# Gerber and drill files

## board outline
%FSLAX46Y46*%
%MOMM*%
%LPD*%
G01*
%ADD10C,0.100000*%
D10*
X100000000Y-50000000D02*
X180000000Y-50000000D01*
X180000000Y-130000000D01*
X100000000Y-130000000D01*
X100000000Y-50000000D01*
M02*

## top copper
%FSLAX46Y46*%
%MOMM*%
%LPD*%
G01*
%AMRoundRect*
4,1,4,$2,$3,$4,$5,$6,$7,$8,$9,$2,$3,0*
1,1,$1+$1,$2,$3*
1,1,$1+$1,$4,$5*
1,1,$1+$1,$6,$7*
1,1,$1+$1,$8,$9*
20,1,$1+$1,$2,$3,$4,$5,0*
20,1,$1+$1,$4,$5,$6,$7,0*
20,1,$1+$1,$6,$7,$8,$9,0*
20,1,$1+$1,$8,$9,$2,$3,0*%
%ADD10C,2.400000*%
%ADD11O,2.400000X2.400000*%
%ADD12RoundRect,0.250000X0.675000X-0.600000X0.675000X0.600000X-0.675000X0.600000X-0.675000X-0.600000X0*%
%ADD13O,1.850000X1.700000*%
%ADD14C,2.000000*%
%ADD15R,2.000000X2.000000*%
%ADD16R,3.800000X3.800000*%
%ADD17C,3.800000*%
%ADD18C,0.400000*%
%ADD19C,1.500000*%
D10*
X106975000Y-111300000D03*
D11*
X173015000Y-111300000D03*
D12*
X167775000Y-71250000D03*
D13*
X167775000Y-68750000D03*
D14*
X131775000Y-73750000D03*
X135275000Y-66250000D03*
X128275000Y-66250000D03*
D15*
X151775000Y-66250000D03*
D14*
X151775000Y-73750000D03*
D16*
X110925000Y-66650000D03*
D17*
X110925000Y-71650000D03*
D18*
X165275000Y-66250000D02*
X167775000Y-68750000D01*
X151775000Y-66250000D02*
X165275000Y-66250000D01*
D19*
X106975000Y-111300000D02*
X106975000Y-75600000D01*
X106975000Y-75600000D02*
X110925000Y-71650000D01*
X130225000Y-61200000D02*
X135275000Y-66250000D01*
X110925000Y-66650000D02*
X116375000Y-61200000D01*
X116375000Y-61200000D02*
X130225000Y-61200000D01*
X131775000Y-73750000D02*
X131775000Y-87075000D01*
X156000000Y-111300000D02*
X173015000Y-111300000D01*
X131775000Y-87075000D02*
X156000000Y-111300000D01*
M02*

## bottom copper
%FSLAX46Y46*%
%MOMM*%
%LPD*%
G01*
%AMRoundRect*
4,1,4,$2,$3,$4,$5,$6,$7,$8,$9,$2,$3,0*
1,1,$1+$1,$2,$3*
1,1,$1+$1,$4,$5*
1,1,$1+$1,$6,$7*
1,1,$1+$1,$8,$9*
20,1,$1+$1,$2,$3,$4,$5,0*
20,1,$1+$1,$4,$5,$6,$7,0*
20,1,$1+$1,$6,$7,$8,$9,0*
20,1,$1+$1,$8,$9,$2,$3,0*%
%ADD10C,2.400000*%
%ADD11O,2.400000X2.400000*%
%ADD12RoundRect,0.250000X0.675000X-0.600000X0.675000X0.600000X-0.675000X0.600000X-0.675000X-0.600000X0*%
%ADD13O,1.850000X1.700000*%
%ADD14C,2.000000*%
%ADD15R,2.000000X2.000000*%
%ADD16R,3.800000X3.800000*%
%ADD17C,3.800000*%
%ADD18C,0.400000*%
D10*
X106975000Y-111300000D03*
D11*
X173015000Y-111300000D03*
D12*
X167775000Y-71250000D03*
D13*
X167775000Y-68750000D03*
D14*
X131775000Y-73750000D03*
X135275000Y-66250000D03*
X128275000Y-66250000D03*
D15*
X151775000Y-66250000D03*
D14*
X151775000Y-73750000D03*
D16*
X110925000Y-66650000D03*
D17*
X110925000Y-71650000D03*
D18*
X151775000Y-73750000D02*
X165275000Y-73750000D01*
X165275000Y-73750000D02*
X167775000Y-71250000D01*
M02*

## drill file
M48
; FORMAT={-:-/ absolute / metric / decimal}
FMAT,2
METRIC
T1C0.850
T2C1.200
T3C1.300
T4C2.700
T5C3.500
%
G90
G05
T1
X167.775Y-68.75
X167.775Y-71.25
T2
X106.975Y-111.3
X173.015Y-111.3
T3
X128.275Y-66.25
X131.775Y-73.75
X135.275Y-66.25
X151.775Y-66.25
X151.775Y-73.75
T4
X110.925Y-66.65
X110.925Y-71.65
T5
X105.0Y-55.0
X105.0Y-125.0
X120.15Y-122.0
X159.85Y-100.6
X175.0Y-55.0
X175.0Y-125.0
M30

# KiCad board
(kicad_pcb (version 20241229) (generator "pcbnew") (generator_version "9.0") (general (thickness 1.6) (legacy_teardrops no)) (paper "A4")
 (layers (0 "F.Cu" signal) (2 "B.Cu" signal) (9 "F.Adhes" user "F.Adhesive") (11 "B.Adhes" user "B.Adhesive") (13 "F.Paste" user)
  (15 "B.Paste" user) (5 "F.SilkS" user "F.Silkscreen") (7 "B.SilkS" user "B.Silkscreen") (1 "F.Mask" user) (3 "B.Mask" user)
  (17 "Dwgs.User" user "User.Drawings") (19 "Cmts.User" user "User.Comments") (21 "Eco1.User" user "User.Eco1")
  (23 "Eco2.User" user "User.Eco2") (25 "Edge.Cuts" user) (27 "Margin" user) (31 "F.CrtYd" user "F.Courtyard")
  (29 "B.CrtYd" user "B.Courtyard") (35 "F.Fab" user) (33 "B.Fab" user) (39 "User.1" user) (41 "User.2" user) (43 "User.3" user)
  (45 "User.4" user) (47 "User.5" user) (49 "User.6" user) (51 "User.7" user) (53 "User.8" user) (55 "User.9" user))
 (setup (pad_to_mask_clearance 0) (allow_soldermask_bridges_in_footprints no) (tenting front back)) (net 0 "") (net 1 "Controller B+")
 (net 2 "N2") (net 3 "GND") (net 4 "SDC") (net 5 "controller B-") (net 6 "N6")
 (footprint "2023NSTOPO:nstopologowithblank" (layer "F.Cu") (at 154.9 81.3)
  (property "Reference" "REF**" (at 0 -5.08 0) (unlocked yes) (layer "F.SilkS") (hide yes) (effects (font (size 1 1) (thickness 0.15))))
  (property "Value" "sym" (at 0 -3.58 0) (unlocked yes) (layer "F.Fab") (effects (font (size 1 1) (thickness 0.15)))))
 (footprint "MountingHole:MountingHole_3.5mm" (layer "F.Cu") (at 175 125)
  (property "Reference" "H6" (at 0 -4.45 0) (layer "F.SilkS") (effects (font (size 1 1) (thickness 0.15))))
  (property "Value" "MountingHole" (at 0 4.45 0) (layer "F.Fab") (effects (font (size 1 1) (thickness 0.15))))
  (pad "" np_thru_hole circle (at 0 0) (size 3.5 3.5) (drill 3.5) (layers "*.Cu" "*.Mask")))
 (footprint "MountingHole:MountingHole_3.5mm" (layer "F.Cu") (at 159.85 100.6)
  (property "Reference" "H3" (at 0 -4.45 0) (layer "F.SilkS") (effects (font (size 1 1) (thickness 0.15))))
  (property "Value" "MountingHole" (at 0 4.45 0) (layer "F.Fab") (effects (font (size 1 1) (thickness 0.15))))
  (pad "" np_thru_hole circle (at 0 0) (size 3.5 3.5) (drill 3.5) (layers "*.Cu" "*.Mask")))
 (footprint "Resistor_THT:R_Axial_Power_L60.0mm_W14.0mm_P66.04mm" (layer "F.Cu") (at 106.975 111.3)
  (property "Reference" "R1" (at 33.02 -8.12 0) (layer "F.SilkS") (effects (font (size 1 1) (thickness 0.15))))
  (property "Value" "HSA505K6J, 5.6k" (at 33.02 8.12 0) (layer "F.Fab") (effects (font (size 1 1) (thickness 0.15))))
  (pad "1" thru_hole circle (at 0 0) (size 2.4 2.4) (drill 1.2) (layers "*.Cu" "*.Mask") (remove_unused_layers no) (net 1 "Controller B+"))
  (pad "2" thru_hole oval (at 66.04 0) (size 2.4 2.4) (drill 1.2) (layers "*.Cu" "*.Mask") (remove_unused_layers no) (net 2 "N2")))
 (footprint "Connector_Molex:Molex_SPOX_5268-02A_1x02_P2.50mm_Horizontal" (layer "F.Cu") (at 167.775 71.25 90)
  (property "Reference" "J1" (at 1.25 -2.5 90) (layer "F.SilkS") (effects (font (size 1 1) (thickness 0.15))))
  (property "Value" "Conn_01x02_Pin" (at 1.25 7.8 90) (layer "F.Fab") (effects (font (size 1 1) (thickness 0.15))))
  (pad "1" thru_hole roundrect (at 0 0 90) (size 1.7 1.85) (drill 0.85) (layers "*.Cu" "*.Mask") (remove_unused_layers no)
   (roundrect_rratio 0.147059) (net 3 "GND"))
  (pad "2" thru_hole oval (at 2.5 0 90) (size 1.7 1.85) (drill 0.85) (layers "*.Cu" "*.Mask") (remove_unused_layers no) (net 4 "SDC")))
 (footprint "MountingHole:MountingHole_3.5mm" (layer "F.Cu") (at 105 125)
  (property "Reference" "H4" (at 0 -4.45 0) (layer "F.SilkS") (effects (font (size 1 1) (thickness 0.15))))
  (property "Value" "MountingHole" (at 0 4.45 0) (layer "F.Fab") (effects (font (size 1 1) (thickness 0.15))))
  (pad "" np_thru_hole circle (at 0 0) (size 3.5 3.5) (drill 3.5) (layers "*.Cu" "*.Mask")))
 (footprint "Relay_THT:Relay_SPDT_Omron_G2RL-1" (layer "F.Cu") (at 151.775 66.25 -90)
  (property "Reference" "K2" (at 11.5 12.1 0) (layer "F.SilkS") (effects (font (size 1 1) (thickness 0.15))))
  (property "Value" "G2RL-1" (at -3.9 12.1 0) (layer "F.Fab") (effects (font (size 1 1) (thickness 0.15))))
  (pad "11" thru_hole circle (at 7.5 20 270) (size 2 2) (drill 1.3) (layers "*.Cu" "*.Mask") (remove_unused_layers no) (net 2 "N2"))
  (pad "12" thru_hole circle (at 0 16.5 270) (size 2 2) (drill 1.3) (layers "*.Cu" "*.Mask") (remove_unused_layers no)
   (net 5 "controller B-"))
  (pad "14" thru_hole circle (at 0 23.5 270) (size 2 2) (drill 1.3) (layers "*.Cu" "*.Mask") (remove_unused_layers no) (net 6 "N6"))
  (pad "A1" thru_hole rect (at 0 0 270) (size 2 2) (drill 1.3) (layers "*.Cu" "*.Mask") (remove_unused_layers no) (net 4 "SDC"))
  (pad "A2" thru_hole circle (at 7.5 0 270) (size 2 2) (drill 1.3) (layers "*.Cu" "*.Mask") (remove_unused_layers no) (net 3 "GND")))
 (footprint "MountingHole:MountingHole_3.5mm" (layer "F.Cu") (at 105 55)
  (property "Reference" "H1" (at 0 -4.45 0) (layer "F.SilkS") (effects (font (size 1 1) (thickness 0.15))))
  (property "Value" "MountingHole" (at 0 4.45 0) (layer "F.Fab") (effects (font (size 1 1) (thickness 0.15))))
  (pad "" np_thru_hole circle (at 0 0) (size 3.5 3.5) (drill 3.5) (layers "*.Cu" "*.Mask")))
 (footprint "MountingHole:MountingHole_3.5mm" (layer "F.Cu") (at 120.15 122)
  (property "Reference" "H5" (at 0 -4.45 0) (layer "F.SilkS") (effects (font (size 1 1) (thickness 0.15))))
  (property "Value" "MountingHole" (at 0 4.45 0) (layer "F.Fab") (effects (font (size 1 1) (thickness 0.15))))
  (pad "" np_thru_hole circle (at 0 0) (size 3.5 3.5) (drill 3.5) (layers "*.Cu" "*.Mask")))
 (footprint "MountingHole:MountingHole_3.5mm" (layer "F.Cu") (at 175 55)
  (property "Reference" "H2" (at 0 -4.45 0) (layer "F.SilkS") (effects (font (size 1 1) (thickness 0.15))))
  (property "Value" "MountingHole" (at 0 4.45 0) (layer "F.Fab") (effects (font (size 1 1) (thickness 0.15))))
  (pad "" np_thru_hole circle (at 0 0) (size 3.5 3.5) (drill 3.5) (layers "*.Cu" "*.Mask")))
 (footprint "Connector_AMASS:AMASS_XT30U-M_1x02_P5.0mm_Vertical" (layer "F.Cu") (at 110.925 66.65 -90)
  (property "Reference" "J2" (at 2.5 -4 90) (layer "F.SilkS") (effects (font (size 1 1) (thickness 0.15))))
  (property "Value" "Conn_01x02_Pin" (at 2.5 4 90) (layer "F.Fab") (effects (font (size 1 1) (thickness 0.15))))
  (pad "1" thru_hole rect (at 0 0 270) (size 3.8 3.8) (drill 2.7) (layers "*.Cu" "*.Mask") (remove_unused_layers no) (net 5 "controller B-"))
  (pad "2" thru_hole circle (at 5 0 270) (size 3.8 3.8) (drill 2.7) (layers "*.Cu" "*.Mask") (remove_unused_layers no)
   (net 1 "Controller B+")))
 (gr_rect (start 100 50) (end 180 130) (stroke (width 0.1) (type default)) (fill no) (layer "Edge.Cuts"))
 (segment (start 165.275 66.25) (end 167.775 68.75) (width 0.4) (layer "F.Cu") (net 4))
 (segment (start 151.775 66.25) (end 165.275 66.25) (width 0.4) (layer "F.Cu") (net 4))
 (segment (start 151.775 73.75) (end 165.275 73.75) (width 0.4) (layer "B.Cu") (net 3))
 (segment (start 165.275 73.75) (end 167.775 71.25) (width 0.4) (layer "B.Cu") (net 3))
 (segment (start 106.975 111.3) (end 106.975 75.6) (width 1.5) (layer "F.Cu") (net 1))
 (segment (start 106.975 75.6) (end 110.925 71.65) (width 1.5) (layer "F.Cu") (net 1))
 (segment (start 130.225 61.2) (end 135.275 66.25) (width 1.5) (layer "F.Cu") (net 5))
 (segment (start 110.925 66.65) (end 116.375 61.2) (width 1.5) (layer "F.Cu") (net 5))
 (segment (start 116.375 61.2) (end 130.225 61.2) (width 1.5) (layer "F.Cu") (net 5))
 (segment (start 131.775 73.75) (end 131.775 87.075) (width 1.5) (layer "F.Cu") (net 2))
 (segment (start 156 111.3) (end 173.015 111.3) (width 1.5) (layer "F.Cu") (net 2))
 (segment (start 131.775 87.075) (end 156 111.3) (width 1.5) (layer "F.Cu") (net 2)))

